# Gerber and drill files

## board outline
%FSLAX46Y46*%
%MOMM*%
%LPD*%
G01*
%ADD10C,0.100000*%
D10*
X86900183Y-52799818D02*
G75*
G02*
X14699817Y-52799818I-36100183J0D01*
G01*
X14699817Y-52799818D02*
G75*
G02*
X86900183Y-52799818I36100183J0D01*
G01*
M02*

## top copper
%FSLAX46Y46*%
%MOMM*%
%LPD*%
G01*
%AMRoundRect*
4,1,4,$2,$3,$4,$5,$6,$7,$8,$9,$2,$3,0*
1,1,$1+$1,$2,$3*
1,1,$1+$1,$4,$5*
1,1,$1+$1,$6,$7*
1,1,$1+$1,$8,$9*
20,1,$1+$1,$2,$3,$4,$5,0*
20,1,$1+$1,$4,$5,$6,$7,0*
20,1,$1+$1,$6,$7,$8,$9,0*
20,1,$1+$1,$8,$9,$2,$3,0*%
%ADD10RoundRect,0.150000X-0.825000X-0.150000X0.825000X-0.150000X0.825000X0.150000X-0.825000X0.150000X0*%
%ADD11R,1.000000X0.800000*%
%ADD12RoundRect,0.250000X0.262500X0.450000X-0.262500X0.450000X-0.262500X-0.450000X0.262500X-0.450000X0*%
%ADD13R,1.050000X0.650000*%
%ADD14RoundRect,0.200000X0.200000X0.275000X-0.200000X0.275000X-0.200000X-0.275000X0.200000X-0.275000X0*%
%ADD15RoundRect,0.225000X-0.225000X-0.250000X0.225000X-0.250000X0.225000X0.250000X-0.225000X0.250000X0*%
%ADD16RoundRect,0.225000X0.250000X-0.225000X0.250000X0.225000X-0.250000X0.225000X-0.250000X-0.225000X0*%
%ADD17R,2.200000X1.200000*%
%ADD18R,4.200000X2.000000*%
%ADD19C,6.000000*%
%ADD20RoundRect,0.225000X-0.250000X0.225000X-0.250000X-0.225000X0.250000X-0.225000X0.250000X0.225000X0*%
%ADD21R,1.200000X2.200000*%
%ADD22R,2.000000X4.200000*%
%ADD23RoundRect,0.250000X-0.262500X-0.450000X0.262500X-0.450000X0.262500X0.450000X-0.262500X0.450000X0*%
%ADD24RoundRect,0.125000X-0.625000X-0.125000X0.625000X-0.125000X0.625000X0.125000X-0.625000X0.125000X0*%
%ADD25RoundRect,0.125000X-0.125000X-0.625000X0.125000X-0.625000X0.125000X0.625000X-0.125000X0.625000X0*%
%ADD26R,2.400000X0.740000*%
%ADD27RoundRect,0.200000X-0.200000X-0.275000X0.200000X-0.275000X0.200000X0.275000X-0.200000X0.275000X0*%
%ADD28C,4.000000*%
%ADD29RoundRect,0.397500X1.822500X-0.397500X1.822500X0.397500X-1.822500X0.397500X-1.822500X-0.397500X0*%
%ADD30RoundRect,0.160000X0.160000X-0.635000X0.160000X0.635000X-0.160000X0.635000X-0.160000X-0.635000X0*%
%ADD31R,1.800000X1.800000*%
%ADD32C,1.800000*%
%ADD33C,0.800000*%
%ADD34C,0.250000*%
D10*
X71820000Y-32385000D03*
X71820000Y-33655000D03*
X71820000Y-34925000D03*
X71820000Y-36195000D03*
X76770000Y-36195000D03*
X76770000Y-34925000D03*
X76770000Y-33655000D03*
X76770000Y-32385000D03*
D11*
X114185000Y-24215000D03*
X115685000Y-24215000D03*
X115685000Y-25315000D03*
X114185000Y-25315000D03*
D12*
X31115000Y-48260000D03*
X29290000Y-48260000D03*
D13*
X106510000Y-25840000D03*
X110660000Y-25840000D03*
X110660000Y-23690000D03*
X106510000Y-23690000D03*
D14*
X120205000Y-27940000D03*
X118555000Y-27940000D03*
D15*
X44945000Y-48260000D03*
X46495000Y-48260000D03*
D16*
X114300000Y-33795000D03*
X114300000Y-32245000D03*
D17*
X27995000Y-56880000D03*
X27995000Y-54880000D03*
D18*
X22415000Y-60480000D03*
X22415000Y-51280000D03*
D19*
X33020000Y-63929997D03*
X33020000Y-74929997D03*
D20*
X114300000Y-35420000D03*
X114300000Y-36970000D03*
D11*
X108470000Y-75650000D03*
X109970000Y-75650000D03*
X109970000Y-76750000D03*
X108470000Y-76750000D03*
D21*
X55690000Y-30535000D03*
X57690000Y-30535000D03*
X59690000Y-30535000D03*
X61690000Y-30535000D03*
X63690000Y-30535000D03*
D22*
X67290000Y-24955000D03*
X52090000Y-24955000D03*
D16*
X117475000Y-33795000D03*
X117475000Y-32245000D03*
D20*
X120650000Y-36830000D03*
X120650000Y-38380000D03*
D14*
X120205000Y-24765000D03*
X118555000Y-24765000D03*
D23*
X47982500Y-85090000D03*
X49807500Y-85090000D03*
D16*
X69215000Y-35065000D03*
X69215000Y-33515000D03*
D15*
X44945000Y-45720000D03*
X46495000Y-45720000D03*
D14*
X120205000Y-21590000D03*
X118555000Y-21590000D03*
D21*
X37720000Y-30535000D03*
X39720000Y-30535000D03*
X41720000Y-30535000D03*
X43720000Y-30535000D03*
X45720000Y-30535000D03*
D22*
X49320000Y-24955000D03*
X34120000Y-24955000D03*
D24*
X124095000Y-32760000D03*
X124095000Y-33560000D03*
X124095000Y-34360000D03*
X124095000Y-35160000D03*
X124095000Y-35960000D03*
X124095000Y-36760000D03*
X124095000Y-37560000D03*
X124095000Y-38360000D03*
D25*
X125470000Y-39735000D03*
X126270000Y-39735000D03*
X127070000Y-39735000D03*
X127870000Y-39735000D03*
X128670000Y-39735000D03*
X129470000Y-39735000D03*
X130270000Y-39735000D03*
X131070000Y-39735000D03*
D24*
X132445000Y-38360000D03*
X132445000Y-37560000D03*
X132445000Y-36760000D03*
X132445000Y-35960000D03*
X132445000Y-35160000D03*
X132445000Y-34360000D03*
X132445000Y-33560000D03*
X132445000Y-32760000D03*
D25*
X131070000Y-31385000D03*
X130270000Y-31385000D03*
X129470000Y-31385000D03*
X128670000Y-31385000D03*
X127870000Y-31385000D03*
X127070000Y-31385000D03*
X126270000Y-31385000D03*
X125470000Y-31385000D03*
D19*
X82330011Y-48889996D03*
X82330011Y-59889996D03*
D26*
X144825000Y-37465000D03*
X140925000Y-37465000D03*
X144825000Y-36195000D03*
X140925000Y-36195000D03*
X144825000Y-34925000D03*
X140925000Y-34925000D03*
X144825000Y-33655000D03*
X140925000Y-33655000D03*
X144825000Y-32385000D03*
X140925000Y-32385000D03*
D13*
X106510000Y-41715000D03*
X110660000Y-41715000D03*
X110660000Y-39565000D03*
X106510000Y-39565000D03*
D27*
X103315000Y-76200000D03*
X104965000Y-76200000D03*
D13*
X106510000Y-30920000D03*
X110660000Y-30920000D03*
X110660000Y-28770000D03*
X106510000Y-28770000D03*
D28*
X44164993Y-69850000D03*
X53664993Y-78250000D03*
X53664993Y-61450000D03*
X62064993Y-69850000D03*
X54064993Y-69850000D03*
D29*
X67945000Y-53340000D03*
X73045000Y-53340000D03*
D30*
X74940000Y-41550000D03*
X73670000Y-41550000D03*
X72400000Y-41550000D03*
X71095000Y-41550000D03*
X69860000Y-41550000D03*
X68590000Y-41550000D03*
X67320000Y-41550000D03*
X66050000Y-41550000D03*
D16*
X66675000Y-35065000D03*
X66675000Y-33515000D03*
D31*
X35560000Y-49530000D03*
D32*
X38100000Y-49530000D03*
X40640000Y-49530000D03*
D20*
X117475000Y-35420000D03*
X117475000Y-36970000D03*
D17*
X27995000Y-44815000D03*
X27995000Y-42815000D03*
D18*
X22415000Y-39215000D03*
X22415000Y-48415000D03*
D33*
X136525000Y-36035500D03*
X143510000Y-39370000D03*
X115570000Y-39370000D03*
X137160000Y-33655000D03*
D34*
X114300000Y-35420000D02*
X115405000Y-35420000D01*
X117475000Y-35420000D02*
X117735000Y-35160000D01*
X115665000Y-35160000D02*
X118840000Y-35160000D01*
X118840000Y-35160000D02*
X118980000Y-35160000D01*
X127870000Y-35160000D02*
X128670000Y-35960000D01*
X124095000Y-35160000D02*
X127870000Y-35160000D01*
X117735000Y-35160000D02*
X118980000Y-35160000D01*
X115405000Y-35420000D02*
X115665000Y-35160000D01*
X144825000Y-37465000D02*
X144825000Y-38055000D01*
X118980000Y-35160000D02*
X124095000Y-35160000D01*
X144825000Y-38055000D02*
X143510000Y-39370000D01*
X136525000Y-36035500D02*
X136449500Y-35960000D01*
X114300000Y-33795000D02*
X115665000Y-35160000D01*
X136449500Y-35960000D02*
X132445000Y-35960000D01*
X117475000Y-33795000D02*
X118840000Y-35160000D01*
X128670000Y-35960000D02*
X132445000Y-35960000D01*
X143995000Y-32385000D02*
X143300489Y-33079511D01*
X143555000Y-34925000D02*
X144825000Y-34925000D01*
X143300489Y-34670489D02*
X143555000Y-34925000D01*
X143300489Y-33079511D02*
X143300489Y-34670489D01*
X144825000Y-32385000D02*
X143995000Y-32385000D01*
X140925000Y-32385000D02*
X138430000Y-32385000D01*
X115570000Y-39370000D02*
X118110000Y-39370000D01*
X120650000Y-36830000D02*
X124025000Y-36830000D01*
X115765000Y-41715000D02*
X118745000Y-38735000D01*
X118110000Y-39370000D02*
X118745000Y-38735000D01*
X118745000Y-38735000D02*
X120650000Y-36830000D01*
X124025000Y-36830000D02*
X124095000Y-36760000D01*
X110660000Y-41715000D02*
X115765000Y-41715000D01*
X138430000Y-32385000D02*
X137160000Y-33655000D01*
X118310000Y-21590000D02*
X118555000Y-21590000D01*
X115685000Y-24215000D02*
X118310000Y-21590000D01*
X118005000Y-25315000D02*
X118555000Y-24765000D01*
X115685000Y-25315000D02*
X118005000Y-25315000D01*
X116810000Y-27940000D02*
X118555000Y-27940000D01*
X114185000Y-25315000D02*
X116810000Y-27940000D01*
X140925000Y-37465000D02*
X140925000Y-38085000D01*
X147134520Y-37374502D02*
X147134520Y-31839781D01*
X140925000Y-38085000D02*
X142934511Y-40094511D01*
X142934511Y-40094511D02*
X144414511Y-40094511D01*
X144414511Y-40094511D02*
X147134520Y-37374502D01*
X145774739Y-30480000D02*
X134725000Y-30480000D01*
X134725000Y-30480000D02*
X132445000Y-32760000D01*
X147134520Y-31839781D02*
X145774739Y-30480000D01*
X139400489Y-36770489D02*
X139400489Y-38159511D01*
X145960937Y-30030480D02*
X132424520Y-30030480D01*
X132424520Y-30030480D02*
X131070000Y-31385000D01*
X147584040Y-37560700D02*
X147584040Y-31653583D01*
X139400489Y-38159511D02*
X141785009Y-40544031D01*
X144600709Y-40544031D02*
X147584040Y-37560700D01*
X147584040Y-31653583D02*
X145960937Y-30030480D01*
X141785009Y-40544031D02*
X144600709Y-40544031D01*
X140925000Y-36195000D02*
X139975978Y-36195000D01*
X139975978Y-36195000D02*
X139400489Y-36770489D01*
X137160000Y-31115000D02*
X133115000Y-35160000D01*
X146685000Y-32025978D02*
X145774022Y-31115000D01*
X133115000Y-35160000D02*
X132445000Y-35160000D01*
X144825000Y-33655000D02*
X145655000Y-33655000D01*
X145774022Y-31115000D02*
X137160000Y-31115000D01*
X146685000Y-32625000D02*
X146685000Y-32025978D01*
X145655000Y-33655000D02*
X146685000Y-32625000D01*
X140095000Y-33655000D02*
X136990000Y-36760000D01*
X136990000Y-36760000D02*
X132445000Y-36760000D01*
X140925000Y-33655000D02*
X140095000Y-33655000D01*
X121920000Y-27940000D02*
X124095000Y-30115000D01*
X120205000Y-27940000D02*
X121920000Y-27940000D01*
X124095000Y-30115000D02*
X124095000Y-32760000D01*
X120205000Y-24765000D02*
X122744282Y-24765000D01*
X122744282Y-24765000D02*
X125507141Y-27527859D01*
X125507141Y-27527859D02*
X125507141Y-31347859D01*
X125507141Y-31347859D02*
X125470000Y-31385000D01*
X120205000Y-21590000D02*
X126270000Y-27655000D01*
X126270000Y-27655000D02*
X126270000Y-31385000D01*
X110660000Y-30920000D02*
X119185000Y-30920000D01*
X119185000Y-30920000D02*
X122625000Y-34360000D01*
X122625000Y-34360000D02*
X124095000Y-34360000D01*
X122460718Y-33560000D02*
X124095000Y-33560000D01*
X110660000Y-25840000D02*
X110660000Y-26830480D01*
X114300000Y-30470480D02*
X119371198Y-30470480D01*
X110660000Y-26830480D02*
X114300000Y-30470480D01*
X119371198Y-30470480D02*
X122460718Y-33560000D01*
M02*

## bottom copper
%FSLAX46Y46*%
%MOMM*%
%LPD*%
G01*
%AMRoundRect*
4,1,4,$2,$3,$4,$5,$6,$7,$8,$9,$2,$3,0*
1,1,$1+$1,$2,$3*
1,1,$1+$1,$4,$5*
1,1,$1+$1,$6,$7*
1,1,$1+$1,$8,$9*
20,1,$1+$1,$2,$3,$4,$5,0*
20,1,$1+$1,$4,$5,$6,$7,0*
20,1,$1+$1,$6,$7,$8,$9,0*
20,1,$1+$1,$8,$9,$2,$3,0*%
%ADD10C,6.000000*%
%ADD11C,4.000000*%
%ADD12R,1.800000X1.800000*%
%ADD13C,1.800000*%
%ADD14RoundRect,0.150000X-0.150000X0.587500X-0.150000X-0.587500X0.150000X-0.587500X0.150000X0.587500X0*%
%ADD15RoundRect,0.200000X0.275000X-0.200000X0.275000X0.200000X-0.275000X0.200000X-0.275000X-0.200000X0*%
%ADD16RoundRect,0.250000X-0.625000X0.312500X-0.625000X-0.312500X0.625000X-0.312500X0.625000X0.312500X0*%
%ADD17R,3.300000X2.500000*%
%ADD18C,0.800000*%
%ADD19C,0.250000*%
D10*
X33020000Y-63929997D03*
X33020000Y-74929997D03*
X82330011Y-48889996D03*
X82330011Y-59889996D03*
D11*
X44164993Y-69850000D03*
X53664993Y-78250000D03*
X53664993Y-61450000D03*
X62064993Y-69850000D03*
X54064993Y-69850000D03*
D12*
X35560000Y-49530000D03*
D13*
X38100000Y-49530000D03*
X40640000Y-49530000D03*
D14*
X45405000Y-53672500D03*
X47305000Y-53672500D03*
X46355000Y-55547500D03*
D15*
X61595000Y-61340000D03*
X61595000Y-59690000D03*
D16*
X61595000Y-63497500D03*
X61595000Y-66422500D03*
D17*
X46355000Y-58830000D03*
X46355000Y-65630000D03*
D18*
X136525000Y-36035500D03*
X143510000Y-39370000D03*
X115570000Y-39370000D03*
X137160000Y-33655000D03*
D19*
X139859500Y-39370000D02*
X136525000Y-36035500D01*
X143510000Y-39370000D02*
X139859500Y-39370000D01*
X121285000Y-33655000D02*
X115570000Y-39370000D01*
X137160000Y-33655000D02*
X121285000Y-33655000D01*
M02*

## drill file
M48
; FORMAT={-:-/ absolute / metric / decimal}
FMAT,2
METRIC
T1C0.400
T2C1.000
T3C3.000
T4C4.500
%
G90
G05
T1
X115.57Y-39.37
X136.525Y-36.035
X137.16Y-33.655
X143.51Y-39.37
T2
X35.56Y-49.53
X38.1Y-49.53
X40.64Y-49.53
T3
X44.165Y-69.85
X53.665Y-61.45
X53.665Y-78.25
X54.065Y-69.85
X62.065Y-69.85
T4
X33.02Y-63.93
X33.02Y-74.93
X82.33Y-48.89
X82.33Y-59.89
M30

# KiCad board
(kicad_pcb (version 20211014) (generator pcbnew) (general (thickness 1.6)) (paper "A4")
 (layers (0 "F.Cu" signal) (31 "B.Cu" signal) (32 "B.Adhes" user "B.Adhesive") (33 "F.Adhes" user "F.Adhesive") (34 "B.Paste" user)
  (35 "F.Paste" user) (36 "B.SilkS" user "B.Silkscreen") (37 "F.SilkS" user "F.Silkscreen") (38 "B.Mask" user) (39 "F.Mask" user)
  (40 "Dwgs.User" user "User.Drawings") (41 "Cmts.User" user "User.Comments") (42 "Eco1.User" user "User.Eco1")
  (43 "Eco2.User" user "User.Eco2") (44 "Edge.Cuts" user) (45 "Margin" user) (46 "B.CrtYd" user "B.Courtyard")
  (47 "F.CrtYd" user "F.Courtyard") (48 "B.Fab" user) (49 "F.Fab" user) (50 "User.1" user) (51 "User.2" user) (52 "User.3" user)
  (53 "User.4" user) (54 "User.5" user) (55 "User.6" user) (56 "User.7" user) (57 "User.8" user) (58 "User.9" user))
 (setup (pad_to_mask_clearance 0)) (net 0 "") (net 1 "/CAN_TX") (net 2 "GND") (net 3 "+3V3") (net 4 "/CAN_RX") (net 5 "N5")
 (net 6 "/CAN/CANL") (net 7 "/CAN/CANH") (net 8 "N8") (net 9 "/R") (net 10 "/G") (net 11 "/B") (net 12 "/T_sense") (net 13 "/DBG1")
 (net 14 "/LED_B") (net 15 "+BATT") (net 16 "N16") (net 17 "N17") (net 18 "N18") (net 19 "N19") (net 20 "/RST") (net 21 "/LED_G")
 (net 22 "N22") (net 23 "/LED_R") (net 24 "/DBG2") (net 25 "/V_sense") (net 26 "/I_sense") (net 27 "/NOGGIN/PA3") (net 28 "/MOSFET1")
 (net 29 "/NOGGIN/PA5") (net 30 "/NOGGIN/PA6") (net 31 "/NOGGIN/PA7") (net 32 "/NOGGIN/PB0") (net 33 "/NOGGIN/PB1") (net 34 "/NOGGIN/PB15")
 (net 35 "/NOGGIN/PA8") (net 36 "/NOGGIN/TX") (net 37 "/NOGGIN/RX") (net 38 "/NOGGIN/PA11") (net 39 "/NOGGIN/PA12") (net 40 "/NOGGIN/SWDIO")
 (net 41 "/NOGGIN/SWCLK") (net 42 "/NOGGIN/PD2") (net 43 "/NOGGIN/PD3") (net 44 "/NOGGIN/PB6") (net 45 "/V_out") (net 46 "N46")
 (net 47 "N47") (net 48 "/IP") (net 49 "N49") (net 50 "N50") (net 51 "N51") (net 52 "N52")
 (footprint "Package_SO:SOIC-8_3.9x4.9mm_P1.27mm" (layer "F.Cu") (at 74.295 34.29)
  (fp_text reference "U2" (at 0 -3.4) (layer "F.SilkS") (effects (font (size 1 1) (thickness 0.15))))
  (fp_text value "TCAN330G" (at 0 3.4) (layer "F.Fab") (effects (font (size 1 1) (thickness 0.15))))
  (pad "1" smd roundrect (at -2.475 -1.905) (size 1.95 0.6) (layers "F.Cu" "F.Paste" "F.Mask") (roundrect_rratio 0.25) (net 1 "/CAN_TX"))
  (pad "2" smd roundrect (at -2.475 -0.635) (size 1.95 0.6) (layers "F.Cu" "F.Paste" "F.Mask") (roundrect_rratio 0.25) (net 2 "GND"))
  (pad "3" smd roundrect (at -2.475 0.635) (size 1.95 0.6) (layers "F.Cu" "F.Paste" "F.Mask") (roundrect_rratio 0.25) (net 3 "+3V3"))
  (pad "4" smd roundrect (at -2.475 1.905) (size 1.95 0.6) (layers "F.Cu" "F.Paste" "F.Mask") (roundrect_rratio 0.25) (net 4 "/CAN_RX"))
  (pad "5" smd roundrect (at 2.475 1.905) (size 1.95 0.6) (layers "F.Cu" "F.Paste" "F.Mask") (roundrect_rratio 0.25) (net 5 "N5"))
  (pad "6" smd roundrect (at 2.475 0.635) (size 1.95 0.6) (layers "F.Cu" "F.Paste" "F.Mask") (roundrect_rratio 0.25) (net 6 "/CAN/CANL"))
  (pad "7" smd roundrect (at 2.475 -0.635) (size 1.95 0.6) (layers "F.Cu" "F.Paste" "F.Mask") (roundrect_rratio 0.25) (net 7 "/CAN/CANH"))
  (pad "8" smd roundrect (at 2.475 -1.905) (size 1.95 0.6) (layers "F.Cu" "F.Paste" "F.Mask") (roundrect_rratio 0.25) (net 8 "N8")))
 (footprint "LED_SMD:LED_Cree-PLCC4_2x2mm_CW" (layer "F.Cu") (at 114.935 24.765)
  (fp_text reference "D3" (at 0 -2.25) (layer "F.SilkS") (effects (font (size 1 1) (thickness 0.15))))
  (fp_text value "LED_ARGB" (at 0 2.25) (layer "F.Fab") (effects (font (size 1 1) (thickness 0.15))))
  (pad "1" smd rect (at -0.75 -0.55) (size 1 0.8) (layers "F.Cu" "F.Paste" "F.Mask") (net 3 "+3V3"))
  (pad "2" smd rect (at 0.75 -0.55) (size 1 0.8) (layers "F.Cu" "F.Paste" "F.Mask") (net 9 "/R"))
  (pad "3" smd rect (at 0.75 0.55) (size 1 0.8) (layers "F.Cu" "F.Paste" "F.Mask") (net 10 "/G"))
  (pad "4" smd rect (at -0.75 0.55) (size 1 0.8) (layers "F.Cu" "F.Paste" "F.Mask") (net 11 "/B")))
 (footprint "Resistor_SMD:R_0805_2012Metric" (layer "F.Cu") (at 30.2025 48.26 180)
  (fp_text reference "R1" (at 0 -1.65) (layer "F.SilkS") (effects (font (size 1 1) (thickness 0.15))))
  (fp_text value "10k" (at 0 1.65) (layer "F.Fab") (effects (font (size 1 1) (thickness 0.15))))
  (pad "1" smd roundrect (at -0.9125 0 180) (size 1.025 1.4) (layers "F.Cu" "F.Paste" "F.Mask") (roundrect_rratio 0.243902) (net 3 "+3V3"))
  (pad "2" smd roundrect (at 0.9125 0 180) (size 1.025 1.4) (layers "F.Cu" "F.Paste" "F.Mask") (roundrect_rratio 0.243902)
   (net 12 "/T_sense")))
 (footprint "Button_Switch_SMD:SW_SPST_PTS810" (layer "F.Cu") (at 108.585 24.765 180)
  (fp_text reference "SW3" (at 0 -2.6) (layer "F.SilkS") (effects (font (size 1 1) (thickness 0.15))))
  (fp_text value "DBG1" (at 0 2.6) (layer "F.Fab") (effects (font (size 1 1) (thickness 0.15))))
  (pad "1" smd rect (at 2.075 -1.075 180) (size 1.05 0.65) (layers "F.Cu" "F.Paste" "F.Mask") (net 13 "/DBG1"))
  (pad "1" smd rect (at -2.075 -1.075 180) (size 1.05 0.65) (layers "F.Cu" "F.Paste" "F.Mask") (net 13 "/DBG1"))
  (pad "2" smd rect (at -2.075 1.075 180) (size 1.05 0.65) (layers "F.Cu" "F.Paste" "F.Mask") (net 2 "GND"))
  (pad "2" smd rect (at 2.075 1.075 180) (size 1.05 0.65) (layers "F.Cu" "F.Paste" "F.Mask") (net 2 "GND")))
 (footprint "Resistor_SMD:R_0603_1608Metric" (layer "F.Cu") (at 119.38 27.94 180)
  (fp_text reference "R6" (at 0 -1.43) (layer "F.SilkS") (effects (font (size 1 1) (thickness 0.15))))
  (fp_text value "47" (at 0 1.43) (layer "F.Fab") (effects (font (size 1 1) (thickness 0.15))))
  (pad "1" smd roundrect (at -0.825 0 180) (size 0.8 0.95) (layers "F.Cu" "F.Paste" "F.Mask") (roundrect_rratio 0.25) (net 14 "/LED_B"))
  (pad "2" smd roundrect (at 0.825 0 180) (size 0.8 0.95) (layers "F.Cu" "F.Paste" "F.Mask") (roundrect_rratio 0.25) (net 11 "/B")))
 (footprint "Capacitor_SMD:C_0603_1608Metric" (layer "F.Cu") (at 45.72 48.26)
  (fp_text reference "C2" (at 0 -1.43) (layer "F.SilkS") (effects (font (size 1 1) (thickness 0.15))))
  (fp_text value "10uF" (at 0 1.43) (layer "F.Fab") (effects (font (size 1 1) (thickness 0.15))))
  (pad "1" smd roundrect (at -0.775 0) (size 0.9 0.95) (layers "F.Cu" "F.Paste" "F.Mask") (roundrect_rratio 0.25) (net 3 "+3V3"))
  (pad "2" smd roundrect (at 0.775 0) (size 0.9 0.95) (layers "F.Cu" "F.Paste" "F.Mask") (roundrect_rratio 0.25) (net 2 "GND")))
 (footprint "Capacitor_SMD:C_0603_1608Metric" (layer "F.Cu") (at 114.3 33.02 90)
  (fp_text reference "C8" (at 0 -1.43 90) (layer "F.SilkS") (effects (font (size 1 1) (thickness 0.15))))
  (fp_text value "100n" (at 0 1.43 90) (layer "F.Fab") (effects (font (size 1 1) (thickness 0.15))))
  (pad "1" smd roundrect (at -0.775 0 90) (size 0.9 0.95) (layers "F.Cu" "F.Paste" "F.Mask") (roundrect_rratio 0.25) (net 3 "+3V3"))
  (pad "2" smd roundrect (at 0.775 0 90) (size 0.9 0.95) (layers "F.Cu" "F.Paste" "F.Mask") (roundrect_rratio 0.25) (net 2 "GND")))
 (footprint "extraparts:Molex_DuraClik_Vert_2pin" (layer "F.Cu") (at 19.415 55.88 -90)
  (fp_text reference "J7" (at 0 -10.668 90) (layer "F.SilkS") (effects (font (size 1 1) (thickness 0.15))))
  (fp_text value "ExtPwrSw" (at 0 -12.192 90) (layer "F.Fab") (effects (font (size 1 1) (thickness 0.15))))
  (pad "1" smd rect locked (at 1 -8.58 270) (size 1.2 2.2) (layers "F.Cu" "F.Paste" "F.Mask") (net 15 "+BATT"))
  (pad "2" smd rect locked (at -1 -8.58 270) (size 1.2 2.2) (layers "F.Cu" "F.Paste" "F.Mask") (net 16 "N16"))
  (pad "MP" smd rect locked (at 4.6 -3 270) (size 2 4.2) (layers "F.Cu" "F.Paste" "F.Mask"))
  (pad "MP" smd rect locked (at -4.6 -3 270) (size 2 4.2) (layers "F.Cu" "F.Paste" "F.Mask")))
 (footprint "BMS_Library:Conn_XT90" (layer "F.Cu") (at 33.02 63.929997 180)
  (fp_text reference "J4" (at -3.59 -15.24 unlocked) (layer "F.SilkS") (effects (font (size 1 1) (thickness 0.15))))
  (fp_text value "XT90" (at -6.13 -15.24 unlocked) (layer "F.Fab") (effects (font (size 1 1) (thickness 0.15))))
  (pad "1" thru_hole circle (at 0 0 180) (size 6 6) (drill 4.5) (layers *.Cu *.Mask) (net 15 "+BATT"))
  (pad "2" thru_hole circle (at 0 -11 180) (size 6 6) (drill 4.5) (layers *.Cu *.Mask) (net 2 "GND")))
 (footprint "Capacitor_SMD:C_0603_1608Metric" (layer "F.Cu") (at 114.3 36.195 -90)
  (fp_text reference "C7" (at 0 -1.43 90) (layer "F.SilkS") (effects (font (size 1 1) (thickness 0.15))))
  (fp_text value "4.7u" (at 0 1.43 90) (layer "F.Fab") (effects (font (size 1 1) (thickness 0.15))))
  (pad "1" smd roundrect (at -0.775 0 270) (size 0.9 0.95) (layers "F.Cu" "F.Paste" "F.Mask") (roundrect_rratio 0.25) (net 3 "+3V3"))
  (pad "2" smd roundrect (at 0.775 0 270) (size 0.9 0.95) (layers "F.Cu" "F.Paste" "F.Mask") (roundrect_rratio 0.25) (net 2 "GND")))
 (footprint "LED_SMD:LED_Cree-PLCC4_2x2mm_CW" (layer "F.Cu") (at 109.22 76.2)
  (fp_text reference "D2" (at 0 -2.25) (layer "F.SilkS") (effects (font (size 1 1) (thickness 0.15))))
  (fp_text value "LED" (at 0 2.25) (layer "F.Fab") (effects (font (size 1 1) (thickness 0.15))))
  (pad "1" smd rect (at -0.75 -0.55) (size 1 0.8) (layers "F.Cu" "F.Paste" "F.Mask") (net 2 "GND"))
  (pad "2" smd rect (at 0.75 -0.55) (size 1 0.8) (layers "F.Cu" "F.Paste" "F.Mask") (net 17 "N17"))
  (pad "3" smd rect (at 0.75 0.55) (size 1 0.8) (layers "F.Cu" "F.Paste" "F.Mask"))
  (pad "4" smd rect (at -0.75 0.55) (size 1 0.8) (layers "F.Cu" "F.Paste" "F.Mask")))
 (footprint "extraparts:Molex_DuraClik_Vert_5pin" (layer "F.Cu") (at 59.69 21.955 180)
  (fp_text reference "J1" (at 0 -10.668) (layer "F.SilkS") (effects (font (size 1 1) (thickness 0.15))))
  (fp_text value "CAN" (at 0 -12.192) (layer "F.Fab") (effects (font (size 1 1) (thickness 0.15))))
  (pad "1" smd rect locked (at 4 -8.58 180) (size 1.2 2.2) (layers "F.Cu" "F.Paste" "F.Mask") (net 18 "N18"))
  (pad "2" smd rect locked (at 2 -8.58 180) (size 1.2 2.2) (layers "F.Cu" "F.Paste" "F.Mask") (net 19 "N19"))
  (pad "3" smd rect locked (at 0 -8.58 180) (size 1.2 2.2) (layers "F.Cu" "F.Paste" "F.Mask") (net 2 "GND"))
  (pad "4" smd rect locked (at -2 -8.58 180) (size 1.2 2.2) (layers "F.Cu" "F.Paste" "F.Mask") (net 7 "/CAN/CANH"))
  (pad "5" smd rect locked (at -4 -8.58 180) (size 1.2 2.2) (layers "F.Cu" "F.Paste" "F.Mask") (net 6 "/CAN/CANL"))
  (pad "MP" smd rect locked (at -7.6 -3 180) (size 2 4.2) (layers "F.Cu" "F.Paste" "F.Mask"))
  (pad "MP" smd rect locked (at 7.6 -3 180) (size 2 4.2) (layers "F.Cu" "F.Paste" "F.Mask")))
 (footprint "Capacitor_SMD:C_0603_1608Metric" (layer "F.Cu") (at 117.475 33.02 90)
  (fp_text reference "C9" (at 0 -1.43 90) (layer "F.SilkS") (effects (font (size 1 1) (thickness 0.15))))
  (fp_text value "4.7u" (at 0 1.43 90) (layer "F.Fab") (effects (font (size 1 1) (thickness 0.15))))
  (pad "1" smd roundrect (at -0.775 0 90) (size 0.9 0.95) (layers "F.Cu" "F.Paste" "F.Mask") (roundrect_rratio 0.25) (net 3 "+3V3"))
  (pad "2" smd roundrect (at 0.775 0 90) (size 0.9 0.95) (layers "F.Cu" "F.Paste" "F.Mask") (roundrect_rratio 0.25) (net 2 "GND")))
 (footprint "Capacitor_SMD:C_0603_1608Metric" (layer "F.Cu") (at 120.65 37.605 -90)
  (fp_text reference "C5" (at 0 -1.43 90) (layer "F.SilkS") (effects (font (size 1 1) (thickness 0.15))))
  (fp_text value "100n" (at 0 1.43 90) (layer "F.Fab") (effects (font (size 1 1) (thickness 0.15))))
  (pad "1" smd roundrect (at -0.775 0 270) (size 0.9 0.95) (layers "F.Cu" "F.Paste" "F.Mask") (roundrect_rratio 0.25) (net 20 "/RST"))
  (pad "2" smd roundrect (at 0.775 0 270) (size 0.9 0.95) (layers "F.Cu" "F.Paste" "F.Mask") (roundrect_rratio 0.25) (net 2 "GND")))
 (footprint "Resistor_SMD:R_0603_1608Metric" (layer "F.Cu") (at 119.38 24.765 180)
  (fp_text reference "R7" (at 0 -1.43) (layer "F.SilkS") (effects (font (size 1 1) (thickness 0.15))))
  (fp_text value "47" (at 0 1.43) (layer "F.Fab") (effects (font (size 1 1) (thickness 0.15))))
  (pad "1" smd roundrect (at -0.825 0 180) (size 0.8 0.95) (layers "F.Cu" "F.Paste" "F.Mask") (roundrect_rratio 0.25) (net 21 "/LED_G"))
  (pad "2" smd roundrect (at 0.825 0 180) (size 0.8 0.95) (layers "F.Cu" "F.Paste" "F.Mask") (roundrect_rratio 0.25) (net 10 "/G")))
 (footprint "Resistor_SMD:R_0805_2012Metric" (layer "F.Cu") (at 48.895 85.09)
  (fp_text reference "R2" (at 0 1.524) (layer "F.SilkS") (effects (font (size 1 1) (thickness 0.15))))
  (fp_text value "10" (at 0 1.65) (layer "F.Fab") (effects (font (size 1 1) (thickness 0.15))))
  (pad "1" smd roundrect (at -0.9125 0) (size 1.025 1.4) (layers "F.Cu" "F.Paste" "F.Mask") (roundrect_rratio 0.243902) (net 15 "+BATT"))
  (pad "2" smd roundrect (at 0.9125 0) (size 1.025 1.4) (layers "F.Cu" "F.Paste" "F.Mask") (roundrect_rratio 0.243902) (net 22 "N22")))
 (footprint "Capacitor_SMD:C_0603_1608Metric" (layer "F.Cu") (at 69.215 34.29 90)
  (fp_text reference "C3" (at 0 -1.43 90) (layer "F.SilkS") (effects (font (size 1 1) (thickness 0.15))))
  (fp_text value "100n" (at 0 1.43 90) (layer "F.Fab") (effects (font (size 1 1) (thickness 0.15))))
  (pad "1" smd roundrect (at -0.775 0 90) (size 0.9 0.95) (layers "F.Cu" "F.Paste" "F.Mask") (roundrect_rratio 0.25) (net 3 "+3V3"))
  (pad "2" smd roundrect (at 0.775 0 90) (size 0.9 0.95) (layers "F.Cu" "F.Paste" "F.Mask") (roundrect_rratio 0.25) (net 2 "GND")))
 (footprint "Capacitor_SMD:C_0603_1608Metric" (layer "F.Cu") (at 45.72 45.72)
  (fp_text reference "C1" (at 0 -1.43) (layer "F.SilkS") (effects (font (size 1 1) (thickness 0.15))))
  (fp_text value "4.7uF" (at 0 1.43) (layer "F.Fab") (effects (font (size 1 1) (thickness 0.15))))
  (pad "1" smd roundrect (at -0.775 0) (size 0.9 0.95) (layers "F.Cu" "F.Paste" "F.Mask") (roundrect_rratio 0.25) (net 16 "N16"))
  (pad "2" smd roundrect (at 0.775 0) (size 0.9 0.95) (layers "F.Cu" "F.Paste" "F.Mask") (roundrect_rratio 0.25) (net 2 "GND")))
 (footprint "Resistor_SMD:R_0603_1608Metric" (layer "F.Cu") (at 119.38 21.59 180)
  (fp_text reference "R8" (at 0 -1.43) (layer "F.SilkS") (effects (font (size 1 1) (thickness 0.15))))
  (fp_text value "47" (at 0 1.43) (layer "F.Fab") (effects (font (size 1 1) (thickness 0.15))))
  (pad "1" smd roundrect (at -0.825 0 180) (size 0.8 0.95) (layers "F.Cu" "F.Paste" "F.Mask") (roundrect_rratio 0.25) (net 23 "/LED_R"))
  (pad "2" smd roundrect (at 0.825 0 180) (size 0.8 0.95) (layers "F.Cu" "F.Paste" "F.Mask") (roundrect_rratio 0.25) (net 9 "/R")))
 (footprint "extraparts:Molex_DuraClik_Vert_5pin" (layer "F.Cu") (at 41.72 21.955 180)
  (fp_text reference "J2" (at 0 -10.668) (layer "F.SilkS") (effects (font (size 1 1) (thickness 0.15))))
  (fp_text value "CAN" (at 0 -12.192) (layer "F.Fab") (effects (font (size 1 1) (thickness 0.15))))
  (pad "1" smd rect locked (at 4 -8.58 180) (size 1.2 2.2) (layers "F.Cu" "F.Paste" "F.Mask") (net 18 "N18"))
  (pad "2" smd rect locked (at 2 -8.58 180) (size 1.2 2.2) (layers "F.Cu" "F.Paste" "F.Mask") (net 19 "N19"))
  (pad "3" smd rect locked (at 0 -8.58 180) (size 1.2 2.2) (layers "F.Cu" "F.Paste" "F.Mask") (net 2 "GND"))
  (pad "4" smd rect locked (at -2 -8.58 180) (size 1.2 2.2) (layers "F.Cu" "F.Paste" "F.Mask") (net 7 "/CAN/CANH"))
  (pad "5" smd rect locked (at -4 -8.58 180) (size 1.2 2.2) (layers "F.Cu" "F.Paste" "F.Mask") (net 6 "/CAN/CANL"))
  (pad "MP" smd rect locked (at -7.6 -3 180) (size 2 4.2) (layers "F.Cu" "F.Paste" "F.Mask"))
  (pad "MP" smd rect locked (at 7.6 -3 180) (size 2 4.2) (layers "F.Cu" "F.Paste" "F.Mask")))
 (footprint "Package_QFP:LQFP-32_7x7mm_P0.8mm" (layer "F.Cu") (at 128.27 35.56)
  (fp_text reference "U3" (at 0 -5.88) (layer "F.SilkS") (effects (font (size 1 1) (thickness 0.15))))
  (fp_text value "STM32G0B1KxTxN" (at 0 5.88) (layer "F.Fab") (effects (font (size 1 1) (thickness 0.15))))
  (pad "1" smd roundrect (at -4.175 -2.8) (size 1.5 0.5) (layers "F.Cu" "F.Paste" "F.Mask") (roundrect_rratio 0.25) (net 14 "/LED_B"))
  (pad "2" smd roundrect (at -4.175 -2) (size 1.5 0.5) (layers "F.Cu" "F.Paste" "F.Mask") (roundrect_rratio 0.25) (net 13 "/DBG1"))
  (pad "3" smd roundrect (at -4.175 -1.2) (size 1.5 0.5) (layers "F.Cu" "F.Paste" "F.Mask") (roundrect_rratio 0.25) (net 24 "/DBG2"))
  (pad "4" smd roundrect (at -4.175 -0.4) (size 1.5 0.5) (layers "F.Cu" "F.Paste" "F.Mask") (roundrect_rratio 0.25) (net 3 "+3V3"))
  (pad "5" smd roundrect (at -4.175 0.4) (size 1.5 0.5) (layers "F.Cu" "F.Paste" "F.Mask") (roundrect_rratio 0.25) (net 2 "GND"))
  (pad "6" smd roundrect (at -4.175 1.2) (size 1.5 0.5) (layers "F.Cu" "F.Paste" "F.Mask") (roundrect_rratio 0.25) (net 20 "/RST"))
  (pad "7" smd roundrect (at -4.175 2) (size 1.5 0.5) (layers "F.Cu" "F.Paste" "F.Mask") (roundrect_rratio 0.25) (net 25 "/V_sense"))
  (pad "8" smd roundrect (at -4.175 2.8) (size 1.5 0.5) (layers "F.Cu" "F.Paste" "F.Mask") (roundrect_rratio 0.25) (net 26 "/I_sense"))
  (pad "9" smd roundrect (at -2.8 4.175) (size 0.5 1.5) (layers "F.Cu" "F.Paste" "F.Mask") (roundrect_rratio 0.25) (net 12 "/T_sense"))
  (pad "10" smd roundrect (at -2 4.175) (size 0.5 1.5) (layers "F.Cu" "F.Paste" "F.Mask") (roundrect_rratio 0.25) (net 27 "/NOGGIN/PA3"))
  (pad "11" smd roundrect (at -1.2 4.175) (size 0.5 1.5) (layers "F.Cu" "F.Paste" "F.Mask") (roundrect_rratio 0.25) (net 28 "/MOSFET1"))
  (pad "12" smd roundrect (at -0.4 4.175) (size 0.5 1.5) (layers "F.Cu" "F.Paste" "F.Mask") (roundrect_rratio 0.25) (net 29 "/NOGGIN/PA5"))
  (pad "13" smd roundrect (at 0.4 4.175) (size 0.5 1.5) (layers "F.Cu" "F.Paste" "F.Mask") (roundrect_rratio 0.25) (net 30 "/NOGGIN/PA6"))
  (pad "14" smd roundrect (at 1.2 4.175) (size 0.5 1.5) (layers "F.Cu" "F.Paste" "F.Mask") (roundrect_rratio 0.25) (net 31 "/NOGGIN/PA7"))
  (pad "15" smd roundrect (at 2 4.175) (size 0.5 1.5) (layers "F.Cu" "F.Paste" "F.Mask") (roundrect_rratio 0.25) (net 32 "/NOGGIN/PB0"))
  (pad "16" smd roundrect (at 2.8 4.175) (size 0.5 1.5) (layers "F.Cu" "F.Paste" "F.Mask") (roundrect_rratio 0.25) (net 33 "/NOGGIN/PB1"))
  (pad "17" smd roundrect (at 4.175 2.8) (size 1.5 0.5) (layers "F.Cu" "F.Paste" "F.Mask") (roundrect_rratio 0.25) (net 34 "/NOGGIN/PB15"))
  (pad "18" smd roundrect (at 4.175 2) (size 1.5 0.5) (layers "F.Cu" "F.Paste" "F.Mask") (roundrect_rratio 0.25) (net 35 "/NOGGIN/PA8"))
  (pad "19" smd roundrect (at 4.175 1.2) (size 1.5 0.5) (layers "F.Cu" "F.Paste" "F.Mask") (roundrect_rratio 0.25) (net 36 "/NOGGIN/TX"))
  (pad "20" smd roundrect (at 4.175 0.4) (size 1.5 0.5) (layers "F.Cu" "F.Paste" "F.Mask") (roundrect_rratio 0.25) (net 3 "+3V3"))
  (pad "21" smd roundrect (at 4.175 -0.4) (size 1.5 0.5) (layers "F.Cu" "F.Paste" "F.Mask") (roundrect_rratio 0.25) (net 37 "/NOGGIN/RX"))
  (pad "22" smd roundrect (at 4.175 -1.2) (size 1.5 0.5) (layers "F.Cu" "F.Paste" "F.Mask") (roundrect_rratio 0.25) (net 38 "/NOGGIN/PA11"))
  (pad "23" smd roundrect (at 4.175 -2) (size 1.5 0.5) (layers "F.Cu" "F.Paste" "F.Mask") (roundrect_rratio 0.25) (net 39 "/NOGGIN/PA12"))
  (pad "24" smd roundrect (at 4.175 -2.8) (size 1.5 0.5) (layers "F.Cu" "F.Paste" "F.Mask") (roundrect_rratio 0.25) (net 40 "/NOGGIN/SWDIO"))
  (pad "25" smd roundrect (at 2.8 -4.175) (size 0.5 1.5) (layers "F.Cu" "F.Paste" "F.Mask") (roundrect_rratio 0.25) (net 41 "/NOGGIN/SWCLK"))
  (pad "26" smd roundrect (at 2 -4.175) (size 0.5 1.5) (layers "F.Cu" "F.Paste" "F.Mask") (roundrect_rratio 0.25) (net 4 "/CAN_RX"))
  (pad "27" smd roundrect (at 1.2 -4.175) (size 0.5 1.5) (layers "F.Cu" "F.Paste" "F.Mask") (roundrect_rratio 0.25) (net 1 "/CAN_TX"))
  (pad "28" smd roundrect (at 0.4 -4.175) (size 0.5 1.5) (layers "F.Cu" "F.Paste" "F.Mask") (roundrect_rratio 0.25) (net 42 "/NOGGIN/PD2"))
  (pad "29" smd roundrect (at -0.4 -4.175) (size 0.5 1.5) (layers "F.Cu" "F.Paste" "F.Mask") (roundrect_rratio 0.25) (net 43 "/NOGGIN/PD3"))
  (pad "30" smd roundrect (at -1.2 -4.175) (size 0.5 1.5) (layers "F.Cu" "F.Paste" "F.Mask") (roundrect_rratio 0.25) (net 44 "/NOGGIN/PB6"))
  (pad "31" smd roundrect (at -2 -4.175) (size 0.5 1.5) (layers "F.Cu" "F.Paste" "F.Mask") (roundrect_rratio 0.25) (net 23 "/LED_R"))
  (pad "32" smd roundrect (at -2.8 -4.175) (size 0.5 1.5) (layers "F.Cu" "F.Paste" "F.Mask") (roundrect_rratio 0.25) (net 21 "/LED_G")))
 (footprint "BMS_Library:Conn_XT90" (layer "F.Cu") (at 82.330011 48.889996 180)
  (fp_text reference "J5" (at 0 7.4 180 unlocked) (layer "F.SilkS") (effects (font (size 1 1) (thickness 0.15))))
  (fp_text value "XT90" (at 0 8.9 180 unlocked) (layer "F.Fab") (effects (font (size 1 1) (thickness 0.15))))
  (pad "1" thru_hole circle (at 0 0 180) (size 6 6) (drill 4.5) (layers *.Cu *.Mask) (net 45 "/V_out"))
  (pad "2" thru_hole circle (at 0 -11 180) (size 6 6) (drill 4.5) (layers *.Cu *.Mask) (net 2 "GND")))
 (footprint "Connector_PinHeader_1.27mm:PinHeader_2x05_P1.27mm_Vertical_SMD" (layer "F.Cu") (at 142.875 34.925 180)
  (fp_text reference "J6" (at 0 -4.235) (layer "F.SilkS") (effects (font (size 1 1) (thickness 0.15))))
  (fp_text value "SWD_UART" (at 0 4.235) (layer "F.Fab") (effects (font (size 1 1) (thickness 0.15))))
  (pad "1" smd rect (at -1.95 -2.54 180) (size 2.4 0.74) (layers "F.Cu" "F.Paste" "F.Mask") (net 3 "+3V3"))
  (pad "2" smd rect (at 1.95 -2.54 180) (size 2.4 0.74) (layers "F.Cu" "F.Paste" "F.Mask") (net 40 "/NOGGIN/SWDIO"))
  (pad "3" smd rect (at -1.95 -1.27 180) (size 2.4 0.74) (layers "F.Cu" "F.Paste" "F.Mask") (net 2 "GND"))
  (pad "4" smd rect (at 1.95 -1.27 180) (size 2.4 0.74) (layers "F.Cu" "F.Paste" "F.Mask") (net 41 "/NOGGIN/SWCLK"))
  (pad "5" smd rect (at -1.95 0 180) (size 2.4 0.74) (layers "F.Cu" "F.Paste" "F.Mask") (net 2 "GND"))
  (pad "6" smd rect (at 1.95 0 180) (size 2.4 0.74) (layers "F.Cu" "F.Paste" "F.Mask") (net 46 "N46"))
  (pad "7" smd rect (at -1.95 1.27 180) (size 2.4 0.74) (layers "F.Cu" "F.Paste" "F.Mask") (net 37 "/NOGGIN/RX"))
  (pad "8" smd rect (at 1.95 1.27 180) (size 2.4 0.74) (layers "F.Cu" "F.Paste" "F.Mask") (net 36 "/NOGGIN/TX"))
  (pad "9" smd rect (at -1.95 2.54 180) (size 2.4 0.74) (layers "F.Cu" "F.Paste" "F.Mask") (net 2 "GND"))
  (pad "10" smd rect (at 1.95 2.54 180) (size 2.4 0.74) (layers "F.Cu" "F.Paste" "F.Mask") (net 20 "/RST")))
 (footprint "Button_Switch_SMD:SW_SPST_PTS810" (layer "F.Cu") (at 108.585 40.64 180)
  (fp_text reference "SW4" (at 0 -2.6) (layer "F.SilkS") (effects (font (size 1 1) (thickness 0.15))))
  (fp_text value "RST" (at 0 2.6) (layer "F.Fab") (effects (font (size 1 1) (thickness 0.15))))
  (pad "1" smd rect (at 2.075 -1.075 180) (size 1.05 0.65) (layers "F.Cu" "F.Paste" "F.Mask") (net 20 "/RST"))
  (pad "1" smd rect (at -2.075 -1.075 180) (size 1.05 0.65) (layers "F.Cu" "F.Paste" "F.Mask") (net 20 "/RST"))
  (pad "2" smd rect (at -2.075 1.075 180) (size 1.05 0.65) (layers "F.Cu" "F.Paste" "F.Mask") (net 2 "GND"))
  (pad "2" smd rect (at 2.075 1.075 180) (size 1.05 0.65) (layers "F.Cu" "F.Paste" "F.Mask") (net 2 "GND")))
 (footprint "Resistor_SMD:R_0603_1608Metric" (layer "F.Cu") (at 104.14 76.2)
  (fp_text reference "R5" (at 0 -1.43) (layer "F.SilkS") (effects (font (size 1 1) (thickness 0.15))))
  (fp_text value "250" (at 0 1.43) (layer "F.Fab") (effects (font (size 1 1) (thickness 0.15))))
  (pad "1" smd roundrect (at -0.825 0) (size 0.8 0.95) (layers "F.Cu" "F.Paste" "F.Mask") (roundrect_rratio 0.25) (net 17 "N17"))
  (pad "2" smd roundrect (at 0.825 0) (size 0.8 0.95) (layers "F.Cu" "F.Paste" "F.Mask") (roundrect_rratio 0.25) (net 45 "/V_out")))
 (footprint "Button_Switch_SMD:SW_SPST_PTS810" (layer "F.Cu") (at 108.585 29.845 180)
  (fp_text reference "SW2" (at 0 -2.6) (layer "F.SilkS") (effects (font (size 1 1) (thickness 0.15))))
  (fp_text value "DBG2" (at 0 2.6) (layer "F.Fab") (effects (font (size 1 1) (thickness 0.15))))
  (pad "1" smd rect (at 2.075 -1.075 180) (size 1.05 0.65) (layers "F.Cu" "F.Paste" "F.Mask") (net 24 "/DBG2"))
  (pad "1" smd rect (at -2.075 -1.075 180) (size 1.05 0.65) (layers "F.Cu" "F.Paste" "F.Mask") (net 24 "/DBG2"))
  (pad "2" smd rect (at -2.075 1.075 180) (size 1.05 0.65) (layers "F.Cu" "F.Paste" "F.Mask") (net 2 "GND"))
  (pad "2" smd rect (at 2.075 1.075 180) (size 1.05 0.65) (layers "F.Cu" "F.Paste" "F.Mask") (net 2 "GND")))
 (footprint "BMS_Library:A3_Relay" (layer "F.Cu") (at 53.664993 69.85)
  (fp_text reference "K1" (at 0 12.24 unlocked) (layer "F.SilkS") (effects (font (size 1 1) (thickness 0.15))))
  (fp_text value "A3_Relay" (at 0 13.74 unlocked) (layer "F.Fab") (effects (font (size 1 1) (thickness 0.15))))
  (pad "30" thru_hole circle (at -9.5 0) (size 4 4) (drill 3) (layers *.Cu *.Mask) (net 15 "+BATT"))
  (pad "85" thru_hole circle (at 0 8.4) (size 4 4) (drill 3) (layers *.Cu *.Mask) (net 22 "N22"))
  (pad "86" thru_hole circle (at 0 -8.4) (size 4 4) (drill 3) (layers *.Cu *.Mask) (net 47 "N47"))
  (pad "87" thru_hole circle (at 8.4 0) (size 4 4) (drill 3) (layers *.Cu *.Mask) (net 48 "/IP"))
  (pad "87a" thru_hole circle (at 0.4 0) (size 4 4) (drill 3) (layers *.Cu *.Mask)))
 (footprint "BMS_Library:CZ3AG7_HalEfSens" (layer "F.Cu") (at 70.495 41.55 90)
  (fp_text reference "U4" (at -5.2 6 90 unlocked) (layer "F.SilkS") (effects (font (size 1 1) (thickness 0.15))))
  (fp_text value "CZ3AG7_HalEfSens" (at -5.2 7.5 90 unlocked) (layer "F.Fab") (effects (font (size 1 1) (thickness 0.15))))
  (pad "1" smd roundrect (at -11.79 -2.55 90) (size 1.59 4.44) (layers "F.Cu" "F.Paste" "F.Mask") (roundrect_rratio 0.25) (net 48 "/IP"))
  (pad "5" smd roundrect (at -11.79 2.55 90) (size 1.59 4.44) (layers "F.Cu" "F.Paste" "F.Mask") (roundrect_rratio 0.25) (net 45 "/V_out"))
  (pad "9" smd roundrect (at 0 4.445 90) (size 1.59 0.64) (layers "F.Cu" "F.Paste" "F.Mask") (roundrect_rratio 0.25) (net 2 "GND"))
  (pad "10" smd roundrect (at 0 3.175 90) (size 1.59 0.64) (layers "F.Cu" "F.Paste" "F.Mask") (roundrect_rratio 0.25) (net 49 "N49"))
  (pad "11" smd roundrect (at 0 1.905 90) (size 1.59 0.64) (layers "F.Cu" "F.Paste" "F.Mask") (roundrect_rratio 0.25) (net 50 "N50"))
  (pad "12" smd roundrect (at 0 0.6 90) (size 1.59 0.64) (layers "F.Cu" "F.Paste" "F.Mask") (roundrect_rratio 0.25) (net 26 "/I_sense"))
  (pad "13" smd roundrect (at 0 -0.635 90) (size 1.59 0.64) (layers "F.Cu" "F.Paste" "F.Mask") (roundrect_rratio 0.25) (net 3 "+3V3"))
  (pad "14" smd roundrect (at 0 -1.905 90) (size 1.59 0.64) (layers "F.Cu" "F.Paste" "F.Mask") (roundrect_rratio 0.25) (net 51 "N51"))
  (pad "15" smd roundrect (at 0 -3.175 90) (size 1.59 0.64) (layers "F.Cu" "F.Paste" "F.Mask") (roundrect_rratio 0.25) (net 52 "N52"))
  (pad "16" smd roundrect (at 0 -4.445 90) (size 1.59 0.64) (layers "F.Cu" "F.Paste" "F.Mask") (roundrect_rratio 0.25) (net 2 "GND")))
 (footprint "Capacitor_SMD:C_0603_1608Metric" (layer "F.Cu") (at 66.675 34.29 90)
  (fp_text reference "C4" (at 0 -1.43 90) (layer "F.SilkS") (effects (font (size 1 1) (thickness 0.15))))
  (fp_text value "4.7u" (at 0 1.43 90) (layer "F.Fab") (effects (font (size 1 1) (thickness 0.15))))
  (pad "1" smd roundrect (at -0.775 0 90) (size 0.9 0.95) (layers "F.Cu" "F.Paste" "F.Mask") (roundrect_rratio 0.25) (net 3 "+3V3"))
  (pad "2" smd roundrect (at 0.775 0 90) (size 0.9 0.95) (layers "F.Cu" "F.Paste" "F.Mask") (roundrect_rratio 0.25) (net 2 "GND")))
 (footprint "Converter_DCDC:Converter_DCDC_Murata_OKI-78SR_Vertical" (layer "F.Cu") (at 35.56 49.53)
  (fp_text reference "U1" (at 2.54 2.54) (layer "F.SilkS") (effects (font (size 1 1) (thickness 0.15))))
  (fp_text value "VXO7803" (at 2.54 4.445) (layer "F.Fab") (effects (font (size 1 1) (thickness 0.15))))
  (pad "1" thru_hole rect (at 0 0) (size 1.8 1.8) (drill 1) (layers *.Cu *.Mask) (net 16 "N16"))
  (pad "2" thru_hole circle (at 2.54 0) (size 1.8 1.8) (drill 1) (layers *.Cu *.Mask) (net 2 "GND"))
  (pad "3" thru_hole circle (at 5.08 0) (size 1.8 1.8) (drill 1) (layers *.Cu *.Mask) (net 3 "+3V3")))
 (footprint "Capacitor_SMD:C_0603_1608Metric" (layer "F.Cu") (at 117.475 36.195 -90)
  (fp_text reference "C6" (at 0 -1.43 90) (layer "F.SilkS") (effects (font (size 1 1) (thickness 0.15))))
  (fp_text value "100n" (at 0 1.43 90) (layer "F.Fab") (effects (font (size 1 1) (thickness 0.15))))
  (pad "1" smd roundrect (at -0.775 0 270) (size 0.9 0.95) (layers "F.Cu" "F.Paste" "F.Mask") (roundrect_rratio 0.25) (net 3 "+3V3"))
  (pad "2" smd roundrect (at 0.775 0 270) (size 0.9 0.95) (layers "F.Cu" "F.Paste" "F.Mask") (roundrect_rratio 0.25) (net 2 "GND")))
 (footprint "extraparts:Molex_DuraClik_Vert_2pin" (layer "F.Cu") (at 19.415 43.815 -90)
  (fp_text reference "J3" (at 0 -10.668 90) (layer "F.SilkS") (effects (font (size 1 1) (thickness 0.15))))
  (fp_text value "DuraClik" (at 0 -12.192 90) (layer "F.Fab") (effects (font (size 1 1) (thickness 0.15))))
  (pad "1" smd rect locked (at 1 -8.58 270) (size 1.2 2.2) (layers "F.Cu" "F.Paste" "F.Mask") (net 12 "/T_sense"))
  (pad "2" smd rect locked (at -1 -8.58 270) (size 1.2 2.2) (layers "F.Cu" "F.Paste" "F.Mask") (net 2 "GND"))
  (pad "MP" smd rect locked (at -4.6 -3 270) (size 2 4.2) (layers "F.Cu" "F.Paste" "F.Mask"))
  (pad "MP" smd rect locked (at 4.6 -3 270) (size 2 4.2) (layers "F.Cu" "F.Paste" "F.Mask")))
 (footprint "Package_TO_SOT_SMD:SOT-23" (layer "B.Cu") (at 46.355 54.61 -90)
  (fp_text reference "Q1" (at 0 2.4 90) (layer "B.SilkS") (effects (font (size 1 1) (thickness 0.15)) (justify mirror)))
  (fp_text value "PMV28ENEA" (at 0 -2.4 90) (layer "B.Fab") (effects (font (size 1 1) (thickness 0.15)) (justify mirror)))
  (pad "1" smd roundrect (at -0.9375 0.95 270) (size 1.475 0.6) (layers "B.Cu" "B.Paste" "B.Mask") (roundrect_rratio 0.25)
   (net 28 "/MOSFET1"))
  (pad "2" smd roundrect (at -0.9375 -0.95 270) (size 1.475 0.6) (layers "B.Cu" "B.Paste" "B.Mask") (roundrect_rratio 0.25) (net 2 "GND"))
  (pad "3" smd roundrect (at 0.9375 0 270) (size 1.475 0.6) (layers "B.Cu" "B.Paste" "B.Mask") (roundrect_rratio 0.25) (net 47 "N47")))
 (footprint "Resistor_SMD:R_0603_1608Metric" (layer "B.Cu") (at 61.595 60.515 90)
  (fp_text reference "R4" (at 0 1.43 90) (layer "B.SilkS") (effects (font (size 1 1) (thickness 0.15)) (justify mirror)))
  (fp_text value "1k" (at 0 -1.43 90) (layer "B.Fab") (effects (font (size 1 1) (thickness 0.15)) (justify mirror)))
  (pad "1" smd roundrect (at -0.825 0 90) (size 0.8 0.95) (layers "B.Cu" "B.Paste" "B.Mask") (roundrect_rratio 0.25) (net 25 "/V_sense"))
  (pad "2" smd roundrect (at 0.825 0 90) (size 0.8 0.95) (layers "B.Cu" "B.Paste" "B.Mask") (roundrect_rratio 0.25) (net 2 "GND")))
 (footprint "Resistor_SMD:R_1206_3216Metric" (layer "B.Cu") (at 61.595 64.96 -90)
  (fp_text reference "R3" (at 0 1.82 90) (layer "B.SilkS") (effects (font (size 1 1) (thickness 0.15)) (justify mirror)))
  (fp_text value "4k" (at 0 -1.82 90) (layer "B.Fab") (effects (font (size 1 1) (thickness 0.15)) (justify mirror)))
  (pad "1" smd roundrect (at -1.4625 0 270) (size 1.125 1.75) (layers "B.Cu" "B.Paste" "B.Mask") (roundrect_rratio 0.222222)
   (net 25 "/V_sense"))
  (pad "2" smd roundrect (at 1.4625 0 270) (size 1.125 1.75) (layers "B.Cu" "B.Paste" "B.Mask") (roundrect_rratio 0.222222) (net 48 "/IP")))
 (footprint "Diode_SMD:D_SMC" (layer "B.Cu") (at 46.355 62.23 -90)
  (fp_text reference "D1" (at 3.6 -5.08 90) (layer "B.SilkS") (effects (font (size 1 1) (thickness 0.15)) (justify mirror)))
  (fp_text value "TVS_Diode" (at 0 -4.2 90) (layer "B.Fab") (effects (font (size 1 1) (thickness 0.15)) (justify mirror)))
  (pad "1" smd rect (at -3.4 0 180) (size 3.3 2.5) (layers "B.Cu" "B.Paste" "B.Mask") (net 47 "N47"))
  (pad "2" smd rect (at 3.4 0 180) (size 3.3 2.5) (layers "B.Cu" "B.Paste" "B.Mask") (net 22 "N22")))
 (gr_circle (center 50.8 52.799818) (end 27.94 80.739818) (layer "Edge.Cuts") (width 0.1) (fill none))
 (segment (start 114.3 35.42) (end 115.405 35.42) (width 0.25) (layer "F.Cu") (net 3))
 (segment (start 117.475 35.42) (end 117.735 35.16) (width 0.25) (layer "F.Cu") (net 3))
 (segment (start 115.665 35.16) (end 118.84 35.16) (width 0.25) (layer "F.Cu") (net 3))
 (segment (start 118.84 35.16) (end 118.98 35.16) (width 0.25) (layer "F.Cu") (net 3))
 (segment (start 127.87 35.16) (end 128.67 35.96) (width 0.25) (layer "F.Cu") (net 3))
 (segment (start 124.095 35.16) (end 127.87 35.16) (width 0.25) (layer "F.Cu") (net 3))
 (segment (start 117.735 35.16) (end 118.98 35.16) (width 0.25) (layer "F.Cu") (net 3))
 (segment (start 115.405 35.42) (end 115.665 35.16) (width 0.25) (layer "F.Cu") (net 3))
 (segment (start 144.825 37.465) (end 144.825 38.055) (width 0.25) (layer "F.Cu") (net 3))
 (segment (start 118.98 35.16) (end 124.095 35.16) (width 0.25) (layer "F.Cu") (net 3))
 (segment (start 144.825 38.055) (end 143.51 39.37) (width 0.25) (layer "F.Cu") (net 3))
 (segment (start 136.525 36.0355) (end 136.4495 35.96) (width 0.25) (layer "F.Cu") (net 3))
 (segment (start 114.3 33.795) (end 115.665 35.16) (width 0.25) (layer "F.Cu") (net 3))
 (segment (start 136.4495 35.96) (end 132.445 35.96) (width 0.25) (layer "F.Cu") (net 3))
 (segment (start 117.475 33.795) (end 118.84 35.16) (width 0.25) (layer "F.Cu") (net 3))
 (segment (start 128.67 35.96) (end 132.445 35.96) (width 0.25) (layer "F.Cu") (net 3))
 (via (at 136.525 36.0355) (size 0.8) (drill 0.4) (layers "F.Cu" "B.Cu") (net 3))
 (via (at 143.51 39.37) (size 0.8) (drill 0.4) (layers "F.Cu" "B.Cu") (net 3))
 (segment (start 139.8595 39.37) (end 136.525 36.0355) (width 0.25) (layer "B.Cu") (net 3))
 (segment (start 143.51 39.37) (end 139.8595 39.37) (width 0.25) (layer "B.Cu") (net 3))
 (segment (start 143.995 32.385) (end 143.300489 33.079511) (width 0.25) (layer "F.Cu") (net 2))
 (segment (start 143.555 34.925) (end 144.825 34.925) (width 0.25) (layer "F.Cu") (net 2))
 (segment (start 143.300489 34.670489) (end 143.555 34.925) (width 0.25) (layer "F.Cu") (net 2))
 (segment (start 143.300489 33.079511) (end 143.300489 34.670489) (width 0.25) (layer "F.Cu") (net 2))
 (segment (start 144.825 32.385) (end 143.995 32.385) (width 0.25) (layer "F.Cu") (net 2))
 (segment (start 140.925 32.385) (end 138.43 32.385) (width 0.25) (layer "F.Cu") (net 20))
 (segment (start 115.57 39.37) (end 118.11 39.37) (width 0.25) (layer "F.Cu") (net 20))
 (segment (start 120.65 36.83) (end 124.025 36.83) (width 0.25) (layer "F.Cu") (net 20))
 (segment (start 115.765 41.715) (end 118.745 38.735) (width 0.25) (layer "F.Cu") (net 20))
 (segment (start 118.11 39.37) (end 118.745 38.735) (width 0.25) (layer "F.Cu") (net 20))
 (segment (start 118.745 38.735) (end 120.65 36.83) (width 0.25) (layer "F.Cu") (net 20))
 (segment (start 124.025 36.83) (end 124.095 36.76) (width 0.25) (layer "F.Cu") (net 20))
 (segment (start 110.66 41.715) (end 115.765 41.715) (width 0.25) (layer "F.Cu") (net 20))
 (segment (start 138.43 32.385) (end 137.16 33.655) (width 0.25) (layer "F.Cu") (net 20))
 (via (at 115.57 39.37) (size 0.8) (drill 0.4) (layers "F.Cu" "B.Cu") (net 20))
 (via (at 137.16 33.655) (size 0.8) (drill 0.4) (layers "F.Cu" "B.Cu") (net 20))
 (segment (start 121.285 33.655) (end 115.57 39.37) (width 0.25) (layer "B.Cu") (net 20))
 (segment (start 137.16 33.655) (end 121.285 33.655) (width 0.25) (layer "B.Cu") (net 20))
 (segment (start 118.31 21.59) (end 118.555 21.59) (width 0.25) (layer "F.Cu") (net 9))
 (segment (start 115.685 24.215) (end 118.31 21.59) (width 0.25) (layer "F.Cu") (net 9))
 (segment (start 118.005 25.315) (end 118.555 24.765) (width 0.25) (layer "F.Cu") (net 10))
 (segment (start 115.685 25.315) (end 118.005 25.315) (width 0.25) (layer "F.Cu") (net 10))
 (segment (start 116.81 27.94) (end 118.555 27.94) (width 0.25) (layer "F.Cu") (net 11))
 (segment (start 114.185 25.315) (end 116.81 27.94) (width 0.25) (layer "F.Cu") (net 11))
 (segment (start 140.925 37.465) (end 140.925 38.085) (width 0.25) (layer "F.Cu") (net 40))
 (segment (start 147.13452 37.374502) (end 147.13452 31.839781) (width 0.25) (layer "F.Cu") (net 40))
 (segment (start 140.925 38.085) (end 142.934511 40.094511) (width 0.25) (layer "F.Cu") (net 40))
 (segment (start 142.934511 40.094511) (end 144.414511 40.094511) (width 0.25) (layer "F.Cu") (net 40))
 (segment (start 144.414511 40.094511) (end 147.13452 37.374502) (width 0.25) (layer "F.Cu") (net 40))
 (segment (start 145.774739 30.48) (end 134.725 30.48) (width 0.25) (layer "F.Cu") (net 40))
 (segment (start 134.725 30.48) (end 132.445 32.76) (width 0.25) (layer "F.Cu") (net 40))
 (segment (start 147.13452 31.839781) (end 145.774739 30.48) (width 0.25) (layer "F.Cu") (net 40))
 (segment (start 139.400489 36.770489) (end 139.400489 38.159511) (width 0.25) (layer "F.Cu") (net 41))
 (segment (start 145.960937 30.03048) (end 132.42452 30.03048) (width 0.25) (layer "F.Cu") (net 41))
 (segment (start 132.42452 30.03048) (end 131.07 31.385) (width 0.25) (layer "F.Cu") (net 41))
 (segment (start 147.58404 37.5607) (end 147.58404 31.653583) (width 0.25) (layer "F.Cu") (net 41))
 (segment (start 139.400489 38.159511) (end 141.785009 40.544031) (width 0.25) (layer "F.Cu") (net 41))
 (segment (start 144.600709 40.544031) (end 147.58404 37.5607) (width 0.25) (layer "F.Cu") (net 41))
 (segment (start 147.58404 31.653583) (end 145.960937 30.03048) (width 0.25) (layer "F.Cu") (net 41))
 (segment (start 141.785009 40.544031) (end 144.600709 40.544031) (width 0.25) (layer "F.Cu") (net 41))
 (segment (start 140.925 36.195) (end 139.975978 36.195) (width 0.25) (layer "F.Cu") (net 41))
 (segment (start 139.975978 36.195) (end 139.400489 36.770489) (width 0.25) (layer "F.Cu") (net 41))
 (segment (start 137.16 31.115) (end 133.115 35.16) (width 0.25) (layer "F.Cu") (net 37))
 (segment (start 146.685 32.025978) (end 145.774022 31.115) (width 0.25) (layer "F.Cu") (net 37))
 (segment (start 133.115 35.16) (end 132.445 35.16) (width 0.25) (layer "F.Cu") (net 37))
 (segment (start 144.825 33.655) (end 145.655 33.655) (width 0.25) (layer "F.Cu") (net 37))
 (segment (start 145.774022 31.115) (end 137.16 31.115) (width 0.25) (layer "F.Cu") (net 37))
 (segment (start 146.685 32.625) (end 146.685 32.025978) (width 0.25) (layer "F.Cu") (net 37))
 (segment (start 145.655 33.655) (end 146.685 32.625) (width 0.25) (layer "F.Cu") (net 37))
 (segment (start 140.095 33.655) (end 136.99 36.76) (width 0.25) (layer "F.Cu") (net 36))
 (segment (start 136.99 36.76) (end 132.445 36.76) (width 0.25) (layer "F.Cu") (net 36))
 (segment (start 140.925 33.655) (end 140.095 33.655) (width 0.25) (layer "F.Cu") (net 36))
 (segment (start 121.92 27.94) (end 124.095 30.115) (width 0.25) (layer "F.Cu") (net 14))
 (segment (start 120.205 27.94) (end 121.92 27.94) (width 0.25) (layer "F.Cu") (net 14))
 (segment (start 124.095 30.115) (end 124.095 32.76) (width 0.25) (layer "F.Cu") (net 14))
 (segment (start 120.205 24.765) (end 122.744282 24.765) (width 0.25) (layer "F.Cu") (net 21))
 (segment (start 122.744282 24.765) (end 125.507141 27.527859) (width 0.25) (layer "F.Cu") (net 21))
 (segment (start 125.507141 27.527859) (end 125.507141 31.347859) (width 0.25) (layer "F.Cu") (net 21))
 (segment (start 125.507141 31.347859) (end 125.47 31.385) (width 0.25) (layer "F.Cu") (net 21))
 (segment (start 120.205 21.59) (end 126.27 27.655) (width 0.25) (layer "F.Cu") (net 23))
 (segment (start 126.27 27.655) (end 126.27 31.385) (width 0.25) (layer "F.Cu") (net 23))
 (segment (start 110.66 30.92) (end 119.185 30.92) (width 0.25) (layer "F.Cu") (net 24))
 (segment (start 119.185 30.92) (end 122.625 34.36) (width 0.25) (layer "F.Cu") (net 24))
 (segment (start 122.625 34.36) (end 124.095 34.36) (width 0.25) (layer "F.Cu") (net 24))
 (segment (start 122.460718 33.56) (end 124.095 33.56) (width 0.25) (layer "F.Cu") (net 13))
 (segment (start 110.66 25.84) (end 110.66 26.83048) (width 0.25) (layer "F.Cu") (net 13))
 (segment (start 114.3 30.47048) (end 119.371198 30.47048) (width 0.25) (layer "F.Cu") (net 13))
 (segment (start 110.66 26.83048) (end 114.3 30.47048) (width 0.25) (layer "F.Cu") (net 13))
 (segment (start 119.371198 30.47048) (end 122.460718 33.56) (width 0.25) (layer "F.Cu") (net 13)))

